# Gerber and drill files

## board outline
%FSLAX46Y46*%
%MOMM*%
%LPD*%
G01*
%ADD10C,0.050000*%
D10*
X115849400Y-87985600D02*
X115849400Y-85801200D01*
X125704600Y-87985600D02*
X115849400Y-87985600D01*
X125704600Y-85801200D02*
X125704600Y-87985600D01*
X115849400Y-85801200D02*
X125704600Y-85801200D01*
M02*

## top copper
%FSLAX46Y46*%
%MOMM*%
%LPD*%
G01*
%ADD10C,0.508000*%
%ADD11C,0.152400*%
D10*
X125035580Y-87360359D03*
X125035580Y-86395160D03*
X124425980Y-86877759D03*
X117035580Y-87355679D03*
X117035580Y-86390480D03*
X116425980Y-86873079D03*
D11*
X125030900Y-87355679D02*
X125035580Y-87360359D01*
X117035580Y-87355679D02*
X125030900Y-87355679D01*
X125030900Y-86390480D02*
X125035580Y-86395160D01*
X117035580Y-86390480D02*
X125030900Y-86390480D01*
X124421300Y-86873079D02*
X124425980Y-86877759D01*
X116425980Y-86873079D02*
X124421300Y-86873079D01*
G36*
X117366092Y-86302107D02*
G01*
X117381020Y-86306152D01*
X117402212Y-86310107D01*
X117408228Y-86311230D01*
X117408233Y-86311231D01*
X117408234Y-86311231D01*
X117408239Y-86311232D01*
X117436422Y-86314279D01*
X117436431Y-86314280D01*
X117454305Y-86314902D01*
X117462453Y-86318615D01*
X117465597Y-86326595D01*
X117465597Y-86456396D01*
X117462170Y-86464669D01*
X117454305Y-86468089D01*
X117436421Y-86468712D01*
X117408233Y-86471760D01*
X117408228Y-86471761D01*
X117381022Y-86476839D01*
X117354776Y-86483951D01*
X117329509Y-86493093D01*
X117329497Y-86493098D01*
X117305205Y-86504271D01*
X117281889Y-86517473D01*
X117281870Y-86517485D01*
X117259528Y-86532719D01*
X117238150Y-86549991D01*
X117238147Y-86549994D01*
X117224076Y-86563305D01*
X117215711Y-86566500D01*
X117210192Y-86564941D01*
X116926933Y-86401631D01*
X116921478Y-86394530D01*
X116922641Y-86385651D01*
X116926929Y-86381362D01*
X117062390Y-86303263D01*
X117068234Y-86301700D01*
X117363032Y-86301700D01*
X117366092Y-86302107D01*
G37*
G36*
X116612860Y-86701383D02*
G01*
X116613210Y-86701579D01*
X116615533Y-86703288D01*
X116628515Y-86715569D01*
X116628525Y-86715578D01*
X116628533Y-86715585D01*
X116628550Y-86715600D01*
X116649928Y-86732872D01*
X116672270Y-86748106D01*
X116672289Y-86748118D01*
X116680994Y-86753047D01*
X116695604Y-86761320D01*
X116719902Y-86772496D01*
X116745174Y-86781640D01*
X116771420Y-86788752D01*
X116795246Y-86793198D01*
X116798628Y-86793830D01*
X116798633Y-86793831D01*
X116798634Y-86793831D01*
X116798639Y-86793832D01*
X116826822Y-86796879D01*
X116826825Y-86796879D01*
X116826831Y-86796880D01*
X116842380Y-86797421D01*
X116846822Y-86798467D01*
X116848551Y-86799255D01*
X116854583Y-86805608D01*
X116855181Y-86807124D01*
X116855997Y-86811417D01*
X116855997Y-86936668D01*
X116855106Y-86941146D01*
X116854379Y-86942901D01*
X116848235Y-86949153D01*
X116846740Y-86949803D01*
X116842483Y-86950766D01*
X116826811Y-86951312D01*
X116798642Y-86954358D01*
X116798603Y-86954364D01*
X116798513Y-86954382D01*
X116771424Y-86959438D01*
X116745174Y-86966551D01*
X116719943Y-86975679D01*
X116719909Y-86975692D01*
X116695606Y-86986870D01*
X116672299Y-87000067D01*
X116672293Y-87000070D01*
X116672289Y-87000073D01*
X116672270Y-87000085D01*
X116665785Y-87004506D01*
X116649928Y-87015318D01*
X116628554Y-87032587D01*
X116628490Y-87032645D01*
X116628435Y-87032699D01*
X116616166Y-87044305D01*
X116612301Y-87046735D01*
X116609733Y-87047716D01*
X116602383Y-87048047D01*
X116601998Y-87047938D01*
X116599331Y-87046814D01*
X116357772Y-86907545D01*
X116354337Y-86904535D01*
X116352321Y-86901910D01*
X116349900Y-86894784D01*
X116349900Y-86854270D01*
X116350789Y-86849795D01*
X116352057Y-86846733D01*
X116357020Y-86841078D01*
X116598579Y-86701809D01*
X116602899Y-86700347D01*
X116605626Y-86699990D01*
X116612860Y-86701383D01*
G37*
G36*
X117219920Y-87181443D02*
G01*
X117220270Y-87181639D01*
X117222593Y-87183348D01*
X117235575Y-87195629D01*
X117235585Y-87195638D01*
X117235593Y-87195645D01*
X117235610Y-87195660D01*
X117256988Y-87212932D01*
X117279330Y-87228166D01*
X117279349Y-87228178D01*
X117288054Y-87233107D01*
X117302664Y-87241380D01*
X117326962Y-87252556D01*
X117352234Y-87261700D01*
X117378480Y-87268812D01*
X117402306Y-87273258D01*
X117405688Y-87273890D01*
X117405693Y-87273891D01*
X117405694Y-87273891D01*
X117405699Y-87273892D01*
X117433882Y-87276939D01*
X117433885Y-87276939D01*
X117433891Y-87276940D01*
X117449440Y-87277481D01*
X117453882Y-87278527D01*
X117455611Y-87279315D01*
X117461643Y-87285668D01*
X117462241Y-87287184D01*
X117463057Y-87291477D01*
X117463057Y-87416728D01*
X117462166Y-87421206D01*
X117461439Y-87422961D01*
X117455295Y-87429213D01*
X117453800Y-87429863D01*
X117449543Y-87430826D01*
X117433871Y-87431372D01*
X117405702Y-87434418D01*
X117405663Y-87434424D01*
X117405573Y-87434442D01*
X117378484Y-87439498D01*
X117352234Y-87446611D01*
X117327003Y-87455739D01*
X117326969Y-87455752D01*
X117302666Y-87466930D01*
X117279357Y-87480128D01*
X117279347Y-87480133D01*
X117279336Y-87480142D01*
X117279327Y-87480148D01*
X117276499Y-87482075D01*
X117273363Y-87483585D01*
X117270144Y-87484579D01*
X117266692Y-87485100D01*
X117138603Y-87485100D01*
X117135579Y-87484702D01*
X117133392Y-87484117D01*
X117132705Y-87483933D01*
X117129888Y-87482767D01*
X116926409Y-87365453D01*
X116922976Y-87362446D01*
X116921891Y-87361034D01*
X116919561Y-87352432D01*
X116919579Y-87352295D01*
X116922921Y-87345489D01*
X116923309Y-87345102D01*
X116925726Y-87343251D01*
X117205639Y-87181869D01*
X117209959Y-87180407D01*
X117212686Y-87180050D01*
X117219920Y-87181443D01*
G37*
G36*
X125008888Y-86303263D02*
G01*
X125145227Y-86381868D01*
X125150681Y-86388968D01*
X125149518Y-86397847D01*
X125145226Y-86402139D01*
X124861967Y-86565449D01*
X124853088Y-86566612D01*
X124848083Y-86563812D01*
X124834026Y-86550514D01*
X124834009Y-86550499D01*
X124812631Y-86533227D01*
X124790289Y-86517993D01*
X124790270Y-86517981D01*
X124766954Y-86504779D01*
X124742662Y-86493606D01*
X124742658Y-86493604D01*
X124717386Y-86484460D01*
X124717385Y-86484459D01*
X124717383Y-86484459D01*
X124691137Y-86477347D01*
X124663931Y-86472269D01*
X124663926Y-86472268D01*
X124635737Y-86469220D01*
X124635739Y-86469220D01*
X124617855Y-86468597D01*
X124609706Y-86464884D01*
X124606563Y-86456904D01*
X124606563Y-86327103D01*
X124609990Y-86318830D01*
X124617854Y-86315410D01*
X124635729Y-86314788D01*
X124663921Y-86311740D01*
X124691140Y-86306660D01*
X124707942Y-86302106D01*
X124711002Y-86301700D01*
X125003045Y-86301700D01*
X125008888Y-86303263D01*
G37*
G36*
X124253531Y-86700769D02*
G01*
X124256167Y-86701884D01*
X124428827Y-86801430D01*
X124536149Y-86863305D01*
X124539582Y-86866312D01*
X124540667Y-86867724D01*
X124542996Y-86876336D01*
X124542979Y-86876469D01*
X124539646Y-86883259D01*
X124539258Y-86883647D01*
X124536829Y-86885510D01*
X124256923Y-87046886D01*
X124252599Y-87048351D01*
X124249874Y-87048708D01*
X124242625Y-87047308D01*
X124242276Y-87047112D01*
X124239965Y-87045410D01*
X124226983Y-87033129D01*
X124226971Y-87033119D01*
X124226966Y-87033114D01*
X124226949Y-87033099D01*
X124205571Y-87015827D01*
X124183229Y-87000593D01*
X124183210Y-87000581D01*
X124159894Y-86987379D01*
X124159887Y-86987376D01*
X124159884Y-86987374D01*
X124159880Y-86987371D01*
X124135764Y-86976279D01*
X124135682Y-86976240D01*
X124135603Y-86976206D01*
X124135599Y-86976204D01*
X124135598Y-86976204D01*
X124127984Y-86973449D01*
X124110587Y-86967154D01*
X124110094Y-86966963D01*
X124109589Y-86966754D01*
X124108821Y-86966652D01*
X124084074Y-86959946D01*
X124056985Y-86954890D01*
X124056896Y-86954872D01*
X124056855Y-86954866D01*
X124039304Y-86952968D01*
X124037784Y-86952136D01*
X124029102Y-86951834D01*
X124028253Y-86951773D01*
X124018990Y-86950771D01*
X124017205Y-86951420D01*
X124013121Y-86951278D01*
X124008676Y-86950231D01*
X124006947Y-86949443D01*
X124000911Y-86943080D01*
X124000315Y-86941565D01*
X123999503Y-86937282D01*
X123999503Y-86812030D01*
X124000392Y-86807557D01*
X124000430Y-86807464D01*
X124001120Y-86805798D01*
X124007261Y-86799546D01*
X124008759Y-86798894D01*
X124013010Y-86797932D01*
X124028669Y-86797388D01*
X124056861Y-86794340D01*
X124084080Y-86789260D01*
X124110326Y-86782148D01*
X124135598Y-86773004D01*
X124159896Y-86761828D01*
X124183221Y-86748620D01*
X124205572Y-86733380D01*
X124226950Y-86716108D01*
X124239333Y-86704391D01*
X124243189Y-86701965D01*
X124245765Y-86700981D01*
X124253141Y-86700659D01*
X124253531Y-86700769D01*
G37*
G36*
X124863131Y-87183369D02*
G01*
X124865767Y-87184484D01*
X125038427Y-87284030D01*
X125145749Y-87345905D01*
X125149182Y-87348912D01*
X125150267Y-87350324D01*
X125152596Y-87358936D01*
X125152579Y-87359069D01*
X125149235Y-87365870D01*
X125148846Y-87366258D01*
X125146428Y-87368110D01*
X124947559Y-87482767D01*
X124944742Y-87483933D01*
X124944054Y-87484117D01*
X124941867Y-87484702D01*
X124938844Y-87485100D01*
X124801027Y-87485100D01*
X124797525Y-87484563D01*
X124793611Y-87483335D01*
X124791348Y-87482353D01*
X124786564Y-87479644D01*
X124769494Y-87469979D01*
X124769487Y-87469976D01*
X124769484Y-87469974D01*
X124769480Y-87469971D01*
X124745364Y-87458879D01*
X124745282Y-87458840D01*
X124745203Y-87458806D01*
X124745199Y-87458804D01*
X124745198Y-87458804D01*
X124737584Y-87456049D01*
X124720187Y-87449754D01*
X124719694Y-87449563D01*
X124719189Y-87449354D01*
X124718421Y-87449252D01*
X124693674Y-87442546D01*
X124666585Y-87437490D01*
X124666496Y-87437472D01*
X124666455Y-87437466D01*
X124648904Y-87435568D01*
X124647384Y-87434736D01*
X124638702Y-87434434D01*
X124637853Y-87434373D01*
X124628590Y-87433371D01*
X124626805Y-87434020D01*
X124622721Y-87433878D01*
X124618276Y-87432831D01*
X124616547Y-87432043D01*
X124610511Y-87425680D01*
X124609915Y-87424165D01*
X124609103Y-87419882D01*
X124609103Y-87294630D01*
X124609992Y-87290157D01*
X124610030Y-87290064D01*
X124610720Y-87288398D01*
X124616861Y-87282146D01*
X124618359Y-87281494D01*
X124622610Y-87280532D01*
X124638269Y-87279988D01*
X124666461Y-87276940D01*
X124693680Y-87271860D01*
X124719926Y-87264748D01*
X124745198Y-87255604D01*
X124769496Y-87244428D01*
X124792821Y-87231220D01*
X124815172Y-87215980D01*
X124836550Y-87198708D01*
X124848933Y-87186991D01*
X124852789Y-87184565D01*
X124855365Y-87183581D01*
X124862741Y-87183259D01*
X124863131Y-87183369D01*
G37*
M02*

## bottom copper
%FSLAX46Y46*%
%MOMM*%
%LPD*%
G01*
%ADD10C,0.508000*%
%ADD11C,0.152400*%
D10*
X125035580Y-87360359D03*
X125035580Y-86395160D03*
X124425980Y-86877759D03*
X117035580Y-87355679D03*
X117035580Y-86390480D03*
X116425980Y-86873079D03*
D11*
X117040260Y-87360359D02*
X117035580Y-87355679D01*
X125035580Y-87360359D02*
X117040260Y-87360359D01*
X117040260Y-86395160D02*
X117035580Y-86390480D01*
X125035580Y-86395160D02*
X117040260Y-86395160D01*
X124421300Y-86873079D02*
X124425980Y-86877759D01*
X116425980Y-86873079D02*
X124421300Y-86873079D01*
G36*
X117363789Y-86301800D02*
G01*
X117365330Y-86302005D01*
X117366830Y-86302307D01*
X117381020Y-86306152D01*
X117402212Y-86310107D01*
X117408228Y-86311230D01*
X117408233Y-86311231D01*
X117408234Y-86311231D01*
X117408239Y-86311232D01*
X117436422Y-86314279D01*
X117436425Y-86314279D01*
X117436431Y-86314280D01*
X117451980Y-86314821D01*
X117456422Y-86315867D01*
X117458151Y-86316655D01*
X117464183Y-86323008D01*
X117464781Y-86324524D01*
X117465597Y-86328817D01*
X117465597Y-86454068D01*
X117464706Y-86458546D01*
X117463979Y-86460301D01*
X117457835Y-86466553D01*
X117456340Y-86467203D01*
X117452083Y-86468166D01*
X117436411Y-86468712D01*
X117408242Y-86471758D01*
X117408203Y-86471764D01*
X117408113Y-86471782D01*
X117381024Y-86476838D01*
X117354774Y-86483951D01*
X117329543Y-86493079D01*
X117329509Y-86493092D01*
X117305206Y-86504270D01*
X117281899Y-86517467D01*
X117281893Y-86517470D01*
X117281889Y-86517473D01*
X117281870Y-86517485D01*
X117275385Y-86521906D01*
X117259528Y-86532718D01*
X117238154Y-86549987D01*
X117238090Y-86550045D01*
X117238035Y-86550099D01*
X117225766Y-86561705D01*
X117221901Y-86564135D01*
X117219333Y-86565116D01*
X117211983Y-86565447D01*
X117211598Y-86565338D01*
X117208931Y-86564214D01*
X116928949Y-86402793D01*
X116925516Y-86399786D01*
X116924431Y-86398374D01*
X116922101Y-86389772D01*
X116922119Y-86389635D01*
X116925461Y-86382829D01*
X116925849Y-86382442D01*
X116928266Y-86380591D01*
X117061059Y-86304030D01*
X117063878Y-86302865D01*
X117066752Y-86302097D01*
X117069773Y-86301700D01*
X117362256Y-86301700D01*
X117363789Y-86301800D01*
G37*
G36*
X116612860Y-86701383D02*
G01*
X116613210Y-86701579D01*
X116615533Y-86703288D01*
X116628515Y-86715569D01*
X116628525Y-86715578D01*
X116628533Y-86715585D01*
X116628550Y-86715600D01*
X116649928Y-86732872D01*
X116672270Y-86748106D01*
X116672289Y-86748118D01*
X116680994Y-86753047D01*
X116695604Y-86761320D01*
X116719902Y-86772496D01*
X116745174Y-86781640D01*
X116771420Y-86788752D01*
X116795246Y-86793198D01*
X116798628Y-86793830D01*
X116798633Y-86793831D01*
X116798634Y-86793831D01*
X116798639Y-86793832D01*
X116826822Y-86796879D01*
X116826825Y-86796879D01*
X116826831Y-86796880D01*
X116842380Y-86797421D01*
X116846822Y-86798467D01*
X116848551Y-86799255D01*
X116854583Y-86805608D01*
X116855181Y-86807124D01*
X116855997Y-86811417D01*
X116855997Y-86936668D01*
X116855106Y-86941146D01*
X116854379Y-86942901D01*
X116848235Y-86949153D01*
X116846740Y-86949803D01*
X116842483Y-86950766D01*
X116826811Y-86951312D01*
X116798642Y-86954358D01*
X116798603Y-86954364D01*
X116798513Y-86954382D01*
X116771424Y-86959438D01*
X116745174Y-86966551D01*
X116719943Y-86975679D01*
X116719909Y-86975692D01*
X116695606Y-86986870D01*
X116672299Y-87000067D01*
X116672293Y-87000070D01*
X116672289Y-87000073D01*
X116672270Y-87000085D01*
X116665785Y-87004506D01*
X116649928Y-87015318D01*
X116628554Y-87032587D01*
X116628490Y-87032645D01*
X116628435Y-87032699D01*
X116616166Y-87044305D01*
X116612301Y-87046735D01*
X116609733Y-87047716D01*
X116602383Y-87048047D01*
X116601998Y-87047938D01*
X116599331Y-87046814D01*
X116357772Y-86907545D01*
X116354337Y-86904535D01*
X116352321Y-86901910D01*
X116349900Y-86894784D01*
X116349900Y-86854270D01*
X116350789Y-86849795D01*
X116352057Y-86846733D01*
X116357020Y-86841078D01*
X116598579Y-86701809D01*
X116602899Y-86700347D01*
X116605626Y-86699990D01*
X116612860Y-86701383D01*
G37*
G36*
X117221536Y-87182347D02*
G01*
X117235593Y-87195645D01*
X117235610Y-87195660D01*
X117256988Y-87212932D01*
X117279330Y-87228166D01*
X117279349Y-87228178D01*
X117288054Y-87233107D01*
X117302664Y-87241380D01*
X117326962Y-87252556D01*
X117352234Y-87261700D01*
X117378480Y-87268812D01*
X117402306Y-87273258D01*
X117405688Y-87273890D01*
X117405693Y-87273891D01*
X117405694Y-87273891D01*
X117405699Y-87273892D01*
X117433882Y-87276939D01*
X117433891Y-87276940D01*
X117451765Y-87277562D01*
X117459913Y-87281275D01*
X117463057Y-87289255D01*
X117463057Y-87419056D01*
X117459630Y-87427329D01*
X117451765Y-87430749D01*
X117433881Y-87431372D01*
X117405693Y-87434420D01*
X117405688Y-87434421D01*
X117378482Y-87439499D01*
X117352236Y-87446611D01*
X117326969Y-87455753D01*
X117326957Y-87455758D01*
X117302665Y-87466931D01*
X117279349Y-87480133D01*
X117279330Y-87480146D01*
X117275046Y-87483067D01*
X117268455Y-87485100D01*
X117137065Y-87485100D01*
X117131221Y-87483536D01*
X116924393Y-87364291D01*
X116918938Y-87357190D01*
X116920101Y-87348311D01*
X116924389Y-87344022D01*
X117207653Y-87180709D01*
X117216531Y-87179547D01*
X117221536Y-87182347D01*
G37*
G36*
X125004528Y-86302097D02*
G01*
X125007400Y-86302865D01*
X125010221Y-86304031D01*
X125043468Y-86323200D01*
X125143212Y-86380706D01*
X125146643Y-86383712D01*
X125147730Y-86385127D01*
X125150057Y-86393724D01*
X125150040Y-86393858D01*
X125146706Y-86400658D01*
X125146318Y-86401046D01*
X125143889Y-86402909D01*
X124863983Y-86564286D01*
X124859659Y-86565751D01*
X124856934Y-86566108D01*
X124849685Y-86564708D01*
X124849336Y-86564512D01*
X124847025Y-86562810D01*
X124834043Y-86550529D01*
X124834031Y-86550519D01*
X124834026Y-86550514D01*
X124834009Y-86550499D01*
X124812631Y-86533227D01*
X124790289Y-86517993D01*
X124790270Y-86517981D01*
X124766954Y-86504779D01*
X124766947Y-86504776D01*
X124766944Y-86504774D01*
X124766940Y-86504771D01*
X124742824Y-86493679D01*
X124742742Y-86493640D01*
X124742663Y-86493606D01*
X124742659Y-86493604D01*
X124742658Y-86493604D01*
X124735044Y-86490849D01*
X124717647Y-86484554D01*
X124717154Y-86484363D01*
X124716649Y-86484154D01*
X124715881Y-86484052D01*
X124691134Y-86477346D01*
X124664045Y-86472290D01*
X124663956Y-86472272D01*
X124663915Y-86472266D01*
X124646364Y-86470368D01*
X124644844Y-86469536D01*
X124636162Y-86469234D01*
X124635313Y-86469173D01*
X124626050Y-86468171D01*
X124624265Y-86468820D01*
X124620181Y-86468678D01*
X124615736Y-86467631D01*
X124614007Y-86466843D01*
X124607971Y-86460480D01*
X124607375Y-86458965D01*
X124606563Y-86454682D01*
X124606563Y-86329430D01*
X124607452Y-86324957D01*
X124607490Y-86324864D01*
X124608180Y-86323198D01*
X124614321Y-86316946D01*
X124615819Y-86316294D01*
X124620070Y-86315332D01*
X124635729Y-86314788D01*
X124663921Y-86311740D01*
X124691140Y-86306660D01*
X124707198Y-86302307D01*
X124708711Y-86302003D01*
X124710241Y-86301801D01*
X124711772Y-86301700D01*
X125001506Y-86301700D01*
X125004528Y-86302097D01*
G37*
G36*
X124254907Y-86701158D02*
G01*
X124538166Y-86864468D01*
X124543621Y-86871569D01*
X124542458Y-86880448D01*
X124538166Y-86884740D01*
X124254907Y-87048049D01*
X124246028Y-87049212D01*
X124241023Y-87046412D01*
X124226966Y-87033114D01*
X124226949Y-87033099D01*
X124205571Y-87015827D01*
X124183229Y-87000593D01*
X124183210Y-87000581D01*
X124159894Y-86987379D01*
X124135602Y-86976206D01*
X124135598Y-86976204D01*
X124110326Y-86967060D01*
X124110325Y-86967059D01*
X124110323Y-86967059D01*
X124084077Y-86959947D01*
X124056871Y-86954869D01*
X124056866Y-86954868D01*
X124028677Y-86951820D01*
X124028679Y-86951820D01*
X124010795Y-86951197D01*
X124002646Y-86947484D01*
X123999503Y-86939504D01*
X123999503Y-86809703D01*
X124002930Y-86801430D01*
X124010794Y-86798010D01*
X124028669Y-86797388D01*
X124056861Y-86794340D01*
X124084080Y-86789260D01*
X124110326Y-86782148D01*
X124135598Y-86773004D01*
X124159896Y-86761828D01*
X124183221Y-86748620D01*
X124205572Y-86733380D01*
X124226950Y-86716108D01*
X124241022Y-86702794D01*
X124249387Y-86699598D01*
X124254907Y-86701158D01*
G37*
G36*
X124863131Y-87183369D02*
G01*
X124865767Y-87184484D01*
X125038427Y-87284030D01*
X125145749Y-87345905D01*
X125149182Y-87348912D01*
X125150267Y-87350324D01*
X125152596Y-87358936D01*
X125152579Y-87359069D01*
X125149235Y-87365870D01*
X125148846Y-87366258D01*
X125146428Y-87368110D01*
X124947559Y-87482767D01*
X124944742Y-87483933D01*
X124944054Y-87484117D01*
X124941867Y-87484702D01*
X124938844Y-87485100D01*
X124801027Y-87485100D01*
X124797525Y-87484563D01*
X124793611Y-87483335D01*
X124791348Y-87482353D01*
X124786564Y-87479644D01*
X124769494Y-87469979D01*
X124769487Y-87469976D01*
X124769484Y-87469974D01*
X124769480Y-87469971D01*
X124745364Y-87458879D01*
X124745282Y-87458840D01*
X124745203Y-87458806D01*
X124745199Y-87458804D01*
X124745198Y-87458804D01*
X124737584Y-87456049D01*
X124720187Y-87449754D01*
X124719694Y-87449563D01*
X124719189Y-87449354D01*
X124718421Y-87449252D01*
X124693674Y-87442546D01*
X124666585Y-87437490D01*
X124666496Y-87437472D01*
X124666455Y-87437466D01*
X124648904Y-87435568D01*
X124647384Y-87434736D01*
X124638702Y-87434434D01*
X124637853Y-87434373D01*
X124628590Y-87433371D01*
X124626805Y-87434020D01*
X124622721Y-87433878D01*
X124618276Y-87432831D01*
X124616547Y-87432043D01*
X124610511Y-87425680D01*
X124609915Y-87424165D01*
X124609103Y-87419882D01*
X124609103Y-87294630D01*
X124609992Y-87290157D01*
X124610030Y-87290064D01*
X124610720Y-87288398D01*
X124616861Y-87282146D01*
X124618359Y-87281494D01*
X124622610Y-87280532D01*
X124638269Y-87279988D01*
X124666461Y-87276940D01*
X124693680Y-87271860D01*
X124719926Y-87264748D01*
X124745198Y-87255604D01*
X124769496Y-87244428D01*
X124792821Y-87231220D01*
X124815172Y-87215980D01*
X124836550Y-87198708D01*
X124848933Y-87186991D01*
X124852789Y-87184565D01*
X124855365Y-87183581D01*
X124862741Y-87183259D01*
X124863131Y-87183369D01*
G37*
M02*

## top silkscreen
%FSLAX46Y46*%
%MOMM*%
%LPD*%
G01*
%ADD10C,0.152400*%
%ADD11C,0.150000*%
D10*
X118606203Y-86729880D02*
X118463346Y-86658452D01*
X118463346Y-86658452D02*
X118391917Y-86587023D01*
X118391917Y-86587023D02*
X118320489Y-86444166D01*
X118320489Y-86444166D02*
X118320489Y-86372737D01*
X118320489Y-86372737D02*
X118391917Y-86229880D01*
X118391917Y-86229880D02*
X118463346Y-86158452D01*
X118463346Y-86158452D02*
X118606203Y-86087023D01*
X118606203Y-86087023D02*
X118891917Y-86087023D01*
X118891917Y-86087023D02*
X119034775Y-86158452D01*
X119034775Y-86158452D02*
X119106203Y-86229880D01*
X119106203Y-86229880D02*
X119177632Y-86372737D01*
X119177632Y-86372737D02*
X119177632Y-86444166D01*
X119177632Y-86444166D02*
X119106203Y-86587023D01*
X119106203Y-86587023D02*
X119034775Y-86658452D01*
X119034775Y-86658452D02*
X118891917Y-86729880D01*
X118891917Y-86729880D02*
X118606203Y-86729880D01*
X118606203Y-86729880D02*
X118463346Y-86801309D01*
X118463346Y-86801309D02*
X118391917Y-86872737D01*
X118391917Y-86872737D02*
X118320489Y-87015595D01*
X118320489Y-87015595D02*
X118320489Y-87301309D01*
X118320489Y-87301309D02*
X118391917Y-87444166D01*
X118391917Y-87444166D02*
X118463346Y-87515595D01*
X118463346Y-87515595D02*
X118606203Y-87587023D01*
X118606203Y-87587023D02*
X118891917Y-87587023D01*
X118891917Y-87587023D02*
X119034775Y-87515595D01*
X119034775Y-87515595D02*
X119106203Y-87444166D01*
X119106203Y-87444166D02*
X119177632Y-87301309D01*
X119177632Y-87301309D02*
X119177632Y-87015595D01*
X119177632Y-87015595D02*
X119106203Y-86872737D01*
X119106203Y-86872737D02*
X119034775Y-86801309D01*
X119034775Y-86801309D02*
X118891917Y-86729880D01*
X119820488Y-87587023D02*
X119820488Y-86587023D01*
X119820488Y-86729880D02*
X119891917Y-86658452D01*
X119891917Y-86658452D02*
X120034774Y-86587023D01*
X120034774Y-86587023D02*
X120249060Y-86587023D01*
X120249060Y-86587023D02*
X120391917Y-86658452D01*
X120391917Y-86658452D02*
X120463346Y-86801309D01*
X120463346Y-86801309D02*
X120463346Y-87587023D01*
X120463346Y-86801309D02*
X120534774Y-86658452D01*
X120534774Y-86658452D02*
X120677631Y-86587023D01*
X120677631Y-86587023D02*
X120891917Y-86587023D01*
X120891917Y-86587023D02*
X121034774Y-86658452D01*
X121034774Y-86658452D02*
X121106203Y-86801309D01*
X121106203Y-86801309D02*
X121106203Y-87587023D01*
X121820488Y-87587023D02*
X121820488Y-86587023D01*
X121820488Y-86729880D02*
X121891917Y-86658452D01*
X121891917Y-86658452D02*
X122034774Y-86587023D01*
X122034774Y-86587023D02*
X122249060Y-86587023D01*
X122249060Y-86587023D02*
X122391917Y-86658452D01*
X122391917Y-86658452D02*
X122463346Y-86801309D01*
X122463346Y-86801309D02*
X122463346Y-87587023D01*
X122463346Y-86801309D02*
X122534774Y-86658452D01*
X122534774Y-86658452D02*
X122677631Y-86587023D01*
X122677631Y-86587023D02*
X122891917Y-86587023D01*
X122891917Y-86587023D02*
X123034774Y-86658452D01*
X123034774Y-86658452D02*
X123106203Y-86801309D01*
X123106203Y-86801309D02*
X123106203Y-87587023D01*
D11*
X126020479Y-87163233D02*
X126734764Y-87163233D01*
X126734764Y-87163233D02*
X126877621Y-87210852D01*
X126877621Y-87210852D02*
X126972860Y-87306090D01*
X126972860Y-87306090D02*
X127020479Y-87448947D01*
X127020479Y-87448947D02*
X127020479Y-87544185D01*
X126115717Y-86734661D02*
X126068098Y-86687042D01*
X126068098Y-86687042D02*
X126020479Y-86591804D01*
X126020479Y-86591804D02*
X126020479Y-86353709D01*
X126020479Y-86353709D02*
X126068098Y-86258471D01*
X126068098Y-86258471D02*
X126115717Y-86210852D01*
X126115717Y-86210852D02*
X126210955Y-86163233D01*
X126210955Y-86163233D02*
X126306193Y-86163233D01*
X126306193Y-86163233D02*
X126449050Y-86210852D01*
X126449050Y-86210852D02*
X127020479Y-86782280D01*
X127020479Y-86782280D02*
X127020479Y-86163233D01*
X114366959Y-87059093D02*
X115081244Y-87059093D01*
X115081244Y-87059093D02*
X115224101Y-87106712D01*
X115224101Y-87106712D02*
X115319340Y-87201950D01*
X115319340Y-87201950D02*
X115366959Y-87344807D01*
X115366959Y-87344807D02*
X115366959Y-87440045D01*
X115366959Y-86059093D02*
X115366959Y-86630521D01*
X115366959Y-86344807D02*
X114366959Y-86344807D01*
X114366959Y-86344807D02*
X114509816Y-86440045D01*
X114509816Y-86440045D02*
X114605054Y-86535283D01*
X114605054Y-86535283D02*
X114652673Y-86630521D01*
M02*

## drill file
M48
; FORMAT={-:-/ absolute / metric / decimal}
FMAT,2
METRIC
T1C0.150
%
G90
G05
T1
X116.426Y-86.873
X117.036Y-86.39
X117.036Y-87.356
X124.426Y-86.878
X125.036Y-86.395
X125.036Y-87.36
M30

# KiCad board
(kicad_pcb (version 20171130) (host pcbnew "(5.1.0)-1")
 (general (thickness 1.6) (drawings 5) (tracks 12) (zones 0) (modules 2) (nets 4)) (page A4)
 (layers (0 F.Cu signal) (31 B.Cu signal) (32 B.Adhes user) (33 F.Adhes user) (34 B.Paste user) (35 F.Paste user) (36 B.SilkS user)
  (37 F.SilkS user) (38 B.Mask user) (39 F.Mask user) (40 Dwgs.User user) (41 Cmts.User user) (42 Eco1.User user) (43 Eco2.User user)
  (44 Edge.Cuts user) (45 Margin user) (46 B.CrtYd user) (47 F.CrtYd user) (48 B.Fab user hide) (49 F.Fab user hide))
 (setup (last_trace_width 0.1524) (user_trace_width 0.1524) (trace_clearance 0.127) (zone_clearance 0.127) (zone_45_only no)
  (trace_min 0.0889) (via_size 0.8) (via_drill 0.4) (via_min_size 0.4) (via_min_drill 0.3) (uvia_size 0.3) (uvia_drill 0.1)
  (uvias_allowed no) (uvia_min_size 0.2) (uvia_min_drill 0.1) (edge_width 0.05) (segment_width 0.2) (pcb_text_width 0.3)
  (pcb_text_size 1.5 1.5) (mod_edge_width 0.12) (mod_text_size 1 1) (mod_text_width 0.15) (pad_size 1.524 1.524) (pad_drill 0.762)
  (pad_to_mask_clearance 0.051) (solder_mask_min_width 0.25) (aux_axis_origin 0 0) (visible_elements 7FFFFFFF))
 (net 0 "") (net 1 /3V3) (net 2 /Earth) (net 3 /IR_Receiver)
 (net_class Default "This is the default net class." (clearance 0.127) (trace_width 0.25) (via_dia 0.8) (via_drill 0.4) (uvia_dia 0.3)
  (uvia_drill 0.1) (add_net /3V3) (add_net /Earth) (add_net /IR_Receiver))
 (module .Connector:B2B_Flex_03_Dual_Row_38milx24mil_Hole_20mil (layer F.Cu) (at 125.01058 86.37016 270)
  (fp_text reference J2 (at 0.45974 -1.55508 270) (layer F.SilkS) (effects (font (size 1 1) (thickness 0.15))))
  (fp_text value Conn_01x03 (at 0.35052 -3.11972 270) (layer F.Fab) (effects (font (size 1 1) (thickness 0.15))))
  (pad 3 thru_hole circle (at 0.990199 -0.025 270) (size 0.508 0.508) (drill 0.15) (layers *.Cu *.Mask) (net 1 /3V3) (zone_connect 2))
  (pad 1 thru_hole circle (at 0.025 -0.025 270) (size 0.508 0.508) (drill 0.15) (layers *.Cu *.Mask) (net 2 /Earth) (zone_connect 2))
  (pad 2 thru_hole circle (at 0.507599 0.5846 270) (size 0.508 0.508) (drill 0.15) (layers *.Cu *.Mask) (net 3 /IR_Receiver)
   (zone_connect 2)))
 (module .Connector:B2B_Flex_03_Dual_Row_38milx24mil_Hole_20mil (layer F.Cu) (at 117.01058 86.36548 270)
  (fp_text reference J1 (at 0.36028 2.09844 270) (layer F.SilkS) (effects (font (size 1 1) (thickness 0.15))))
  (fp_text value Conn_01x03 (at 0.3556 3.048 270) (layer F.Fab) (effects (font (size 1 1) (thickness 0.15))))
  (pad 3 thru_hole circle (at 0.990199 -0.025 270) (size 0.508 0.508) (drill 0.15) (layers *.Cu *.Mask) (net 1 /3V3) (zone_connect 2))
  (pad 1 thru_hole circle (at 0.025 -0.025 270) (size 0.508 0.508) (drill 0.15) (layers *.Cu *.Mask) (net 2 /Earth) (zone_connect 2))
  (pad 2 thru_hole circle (at 0.507599 0.5846 270) (size 0.508 0.508) (drill 0.15) (layers *.Cu *.Mask) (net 3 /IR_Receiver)
   (zone_connect 2)))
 (gr_line (start 115.8494 87.9856) (end 115.8494 85.8012) (layer Edge.Cuts) (width 0.05))
 (gr_line (start 125.7046 87.9856) (end 115.8494 87.9856) (layer Edge.Cuts) (width 0.05))
 (gr_line (start 125.7046 85.8012) (end 125.7046 87.9856) (layer Edge.Cuts) (width 0.05))
 (gr_line (start 115.8494 85.8012) (end 125.7046 85.8012) (layer Edge.Cuts) (width 0.05))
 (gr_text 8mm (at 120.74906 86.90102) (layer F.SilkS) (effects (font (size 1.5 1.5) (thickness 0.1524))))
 (segment (start 125.0309 87.355679) (end 125.03558 87.360359) (width 0.1524) (layer F.Cu) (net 1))
 (segment (start 117.03558 87.355679) (end 125.0309 87.355679) (width 0.1524) (layer F.Cu) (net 1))
 (segment (start 117.04026 87.360359) (end 117.03558 87.355679) (width 0.1524) (layer B.Cu) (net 1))
 (segment (start 125.03558 87.360359) (end 117.04026 87.360359) (width 0.1524) (layer B.Cu) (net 1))
 (segment (start 125.0309 86.39048) (end 125.03558 86.39516) (width 0.1524) (layer F.Cu) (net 2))
 (segment (start 117.03558 86.39048) (end 125.0309 86.39048) (width 0.1524) (layer F.Cu) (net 2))
 (segment (start 117.04026 86.39516) (end 117.03558 86.39048) (width 0.1524) (layer B.Cu) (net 2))
 (segment (start 125.03558 86.39516) (end 117.04026 86.39516) (width 0.1524) (layer B.Cu) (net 2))
 (segment (start 124.4213 86.873079) (end 124.42598 86.877759) (width 0.1524) (layer F.Cu) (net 3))
 (segment (start 116.42598 86.873079) (end 124.4213 86.873079) (width 0.1524) (layer F.Cu) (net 3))
 (segment (start 124.4213 86.873079) (end 124.42598 86.877759) (width 0.1524) (layer B.Cu) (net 3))
 (segment (start 116.42598 86.873079) (end 124.4213 86.873079) (width 0.1524) (layer B.Cu) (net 3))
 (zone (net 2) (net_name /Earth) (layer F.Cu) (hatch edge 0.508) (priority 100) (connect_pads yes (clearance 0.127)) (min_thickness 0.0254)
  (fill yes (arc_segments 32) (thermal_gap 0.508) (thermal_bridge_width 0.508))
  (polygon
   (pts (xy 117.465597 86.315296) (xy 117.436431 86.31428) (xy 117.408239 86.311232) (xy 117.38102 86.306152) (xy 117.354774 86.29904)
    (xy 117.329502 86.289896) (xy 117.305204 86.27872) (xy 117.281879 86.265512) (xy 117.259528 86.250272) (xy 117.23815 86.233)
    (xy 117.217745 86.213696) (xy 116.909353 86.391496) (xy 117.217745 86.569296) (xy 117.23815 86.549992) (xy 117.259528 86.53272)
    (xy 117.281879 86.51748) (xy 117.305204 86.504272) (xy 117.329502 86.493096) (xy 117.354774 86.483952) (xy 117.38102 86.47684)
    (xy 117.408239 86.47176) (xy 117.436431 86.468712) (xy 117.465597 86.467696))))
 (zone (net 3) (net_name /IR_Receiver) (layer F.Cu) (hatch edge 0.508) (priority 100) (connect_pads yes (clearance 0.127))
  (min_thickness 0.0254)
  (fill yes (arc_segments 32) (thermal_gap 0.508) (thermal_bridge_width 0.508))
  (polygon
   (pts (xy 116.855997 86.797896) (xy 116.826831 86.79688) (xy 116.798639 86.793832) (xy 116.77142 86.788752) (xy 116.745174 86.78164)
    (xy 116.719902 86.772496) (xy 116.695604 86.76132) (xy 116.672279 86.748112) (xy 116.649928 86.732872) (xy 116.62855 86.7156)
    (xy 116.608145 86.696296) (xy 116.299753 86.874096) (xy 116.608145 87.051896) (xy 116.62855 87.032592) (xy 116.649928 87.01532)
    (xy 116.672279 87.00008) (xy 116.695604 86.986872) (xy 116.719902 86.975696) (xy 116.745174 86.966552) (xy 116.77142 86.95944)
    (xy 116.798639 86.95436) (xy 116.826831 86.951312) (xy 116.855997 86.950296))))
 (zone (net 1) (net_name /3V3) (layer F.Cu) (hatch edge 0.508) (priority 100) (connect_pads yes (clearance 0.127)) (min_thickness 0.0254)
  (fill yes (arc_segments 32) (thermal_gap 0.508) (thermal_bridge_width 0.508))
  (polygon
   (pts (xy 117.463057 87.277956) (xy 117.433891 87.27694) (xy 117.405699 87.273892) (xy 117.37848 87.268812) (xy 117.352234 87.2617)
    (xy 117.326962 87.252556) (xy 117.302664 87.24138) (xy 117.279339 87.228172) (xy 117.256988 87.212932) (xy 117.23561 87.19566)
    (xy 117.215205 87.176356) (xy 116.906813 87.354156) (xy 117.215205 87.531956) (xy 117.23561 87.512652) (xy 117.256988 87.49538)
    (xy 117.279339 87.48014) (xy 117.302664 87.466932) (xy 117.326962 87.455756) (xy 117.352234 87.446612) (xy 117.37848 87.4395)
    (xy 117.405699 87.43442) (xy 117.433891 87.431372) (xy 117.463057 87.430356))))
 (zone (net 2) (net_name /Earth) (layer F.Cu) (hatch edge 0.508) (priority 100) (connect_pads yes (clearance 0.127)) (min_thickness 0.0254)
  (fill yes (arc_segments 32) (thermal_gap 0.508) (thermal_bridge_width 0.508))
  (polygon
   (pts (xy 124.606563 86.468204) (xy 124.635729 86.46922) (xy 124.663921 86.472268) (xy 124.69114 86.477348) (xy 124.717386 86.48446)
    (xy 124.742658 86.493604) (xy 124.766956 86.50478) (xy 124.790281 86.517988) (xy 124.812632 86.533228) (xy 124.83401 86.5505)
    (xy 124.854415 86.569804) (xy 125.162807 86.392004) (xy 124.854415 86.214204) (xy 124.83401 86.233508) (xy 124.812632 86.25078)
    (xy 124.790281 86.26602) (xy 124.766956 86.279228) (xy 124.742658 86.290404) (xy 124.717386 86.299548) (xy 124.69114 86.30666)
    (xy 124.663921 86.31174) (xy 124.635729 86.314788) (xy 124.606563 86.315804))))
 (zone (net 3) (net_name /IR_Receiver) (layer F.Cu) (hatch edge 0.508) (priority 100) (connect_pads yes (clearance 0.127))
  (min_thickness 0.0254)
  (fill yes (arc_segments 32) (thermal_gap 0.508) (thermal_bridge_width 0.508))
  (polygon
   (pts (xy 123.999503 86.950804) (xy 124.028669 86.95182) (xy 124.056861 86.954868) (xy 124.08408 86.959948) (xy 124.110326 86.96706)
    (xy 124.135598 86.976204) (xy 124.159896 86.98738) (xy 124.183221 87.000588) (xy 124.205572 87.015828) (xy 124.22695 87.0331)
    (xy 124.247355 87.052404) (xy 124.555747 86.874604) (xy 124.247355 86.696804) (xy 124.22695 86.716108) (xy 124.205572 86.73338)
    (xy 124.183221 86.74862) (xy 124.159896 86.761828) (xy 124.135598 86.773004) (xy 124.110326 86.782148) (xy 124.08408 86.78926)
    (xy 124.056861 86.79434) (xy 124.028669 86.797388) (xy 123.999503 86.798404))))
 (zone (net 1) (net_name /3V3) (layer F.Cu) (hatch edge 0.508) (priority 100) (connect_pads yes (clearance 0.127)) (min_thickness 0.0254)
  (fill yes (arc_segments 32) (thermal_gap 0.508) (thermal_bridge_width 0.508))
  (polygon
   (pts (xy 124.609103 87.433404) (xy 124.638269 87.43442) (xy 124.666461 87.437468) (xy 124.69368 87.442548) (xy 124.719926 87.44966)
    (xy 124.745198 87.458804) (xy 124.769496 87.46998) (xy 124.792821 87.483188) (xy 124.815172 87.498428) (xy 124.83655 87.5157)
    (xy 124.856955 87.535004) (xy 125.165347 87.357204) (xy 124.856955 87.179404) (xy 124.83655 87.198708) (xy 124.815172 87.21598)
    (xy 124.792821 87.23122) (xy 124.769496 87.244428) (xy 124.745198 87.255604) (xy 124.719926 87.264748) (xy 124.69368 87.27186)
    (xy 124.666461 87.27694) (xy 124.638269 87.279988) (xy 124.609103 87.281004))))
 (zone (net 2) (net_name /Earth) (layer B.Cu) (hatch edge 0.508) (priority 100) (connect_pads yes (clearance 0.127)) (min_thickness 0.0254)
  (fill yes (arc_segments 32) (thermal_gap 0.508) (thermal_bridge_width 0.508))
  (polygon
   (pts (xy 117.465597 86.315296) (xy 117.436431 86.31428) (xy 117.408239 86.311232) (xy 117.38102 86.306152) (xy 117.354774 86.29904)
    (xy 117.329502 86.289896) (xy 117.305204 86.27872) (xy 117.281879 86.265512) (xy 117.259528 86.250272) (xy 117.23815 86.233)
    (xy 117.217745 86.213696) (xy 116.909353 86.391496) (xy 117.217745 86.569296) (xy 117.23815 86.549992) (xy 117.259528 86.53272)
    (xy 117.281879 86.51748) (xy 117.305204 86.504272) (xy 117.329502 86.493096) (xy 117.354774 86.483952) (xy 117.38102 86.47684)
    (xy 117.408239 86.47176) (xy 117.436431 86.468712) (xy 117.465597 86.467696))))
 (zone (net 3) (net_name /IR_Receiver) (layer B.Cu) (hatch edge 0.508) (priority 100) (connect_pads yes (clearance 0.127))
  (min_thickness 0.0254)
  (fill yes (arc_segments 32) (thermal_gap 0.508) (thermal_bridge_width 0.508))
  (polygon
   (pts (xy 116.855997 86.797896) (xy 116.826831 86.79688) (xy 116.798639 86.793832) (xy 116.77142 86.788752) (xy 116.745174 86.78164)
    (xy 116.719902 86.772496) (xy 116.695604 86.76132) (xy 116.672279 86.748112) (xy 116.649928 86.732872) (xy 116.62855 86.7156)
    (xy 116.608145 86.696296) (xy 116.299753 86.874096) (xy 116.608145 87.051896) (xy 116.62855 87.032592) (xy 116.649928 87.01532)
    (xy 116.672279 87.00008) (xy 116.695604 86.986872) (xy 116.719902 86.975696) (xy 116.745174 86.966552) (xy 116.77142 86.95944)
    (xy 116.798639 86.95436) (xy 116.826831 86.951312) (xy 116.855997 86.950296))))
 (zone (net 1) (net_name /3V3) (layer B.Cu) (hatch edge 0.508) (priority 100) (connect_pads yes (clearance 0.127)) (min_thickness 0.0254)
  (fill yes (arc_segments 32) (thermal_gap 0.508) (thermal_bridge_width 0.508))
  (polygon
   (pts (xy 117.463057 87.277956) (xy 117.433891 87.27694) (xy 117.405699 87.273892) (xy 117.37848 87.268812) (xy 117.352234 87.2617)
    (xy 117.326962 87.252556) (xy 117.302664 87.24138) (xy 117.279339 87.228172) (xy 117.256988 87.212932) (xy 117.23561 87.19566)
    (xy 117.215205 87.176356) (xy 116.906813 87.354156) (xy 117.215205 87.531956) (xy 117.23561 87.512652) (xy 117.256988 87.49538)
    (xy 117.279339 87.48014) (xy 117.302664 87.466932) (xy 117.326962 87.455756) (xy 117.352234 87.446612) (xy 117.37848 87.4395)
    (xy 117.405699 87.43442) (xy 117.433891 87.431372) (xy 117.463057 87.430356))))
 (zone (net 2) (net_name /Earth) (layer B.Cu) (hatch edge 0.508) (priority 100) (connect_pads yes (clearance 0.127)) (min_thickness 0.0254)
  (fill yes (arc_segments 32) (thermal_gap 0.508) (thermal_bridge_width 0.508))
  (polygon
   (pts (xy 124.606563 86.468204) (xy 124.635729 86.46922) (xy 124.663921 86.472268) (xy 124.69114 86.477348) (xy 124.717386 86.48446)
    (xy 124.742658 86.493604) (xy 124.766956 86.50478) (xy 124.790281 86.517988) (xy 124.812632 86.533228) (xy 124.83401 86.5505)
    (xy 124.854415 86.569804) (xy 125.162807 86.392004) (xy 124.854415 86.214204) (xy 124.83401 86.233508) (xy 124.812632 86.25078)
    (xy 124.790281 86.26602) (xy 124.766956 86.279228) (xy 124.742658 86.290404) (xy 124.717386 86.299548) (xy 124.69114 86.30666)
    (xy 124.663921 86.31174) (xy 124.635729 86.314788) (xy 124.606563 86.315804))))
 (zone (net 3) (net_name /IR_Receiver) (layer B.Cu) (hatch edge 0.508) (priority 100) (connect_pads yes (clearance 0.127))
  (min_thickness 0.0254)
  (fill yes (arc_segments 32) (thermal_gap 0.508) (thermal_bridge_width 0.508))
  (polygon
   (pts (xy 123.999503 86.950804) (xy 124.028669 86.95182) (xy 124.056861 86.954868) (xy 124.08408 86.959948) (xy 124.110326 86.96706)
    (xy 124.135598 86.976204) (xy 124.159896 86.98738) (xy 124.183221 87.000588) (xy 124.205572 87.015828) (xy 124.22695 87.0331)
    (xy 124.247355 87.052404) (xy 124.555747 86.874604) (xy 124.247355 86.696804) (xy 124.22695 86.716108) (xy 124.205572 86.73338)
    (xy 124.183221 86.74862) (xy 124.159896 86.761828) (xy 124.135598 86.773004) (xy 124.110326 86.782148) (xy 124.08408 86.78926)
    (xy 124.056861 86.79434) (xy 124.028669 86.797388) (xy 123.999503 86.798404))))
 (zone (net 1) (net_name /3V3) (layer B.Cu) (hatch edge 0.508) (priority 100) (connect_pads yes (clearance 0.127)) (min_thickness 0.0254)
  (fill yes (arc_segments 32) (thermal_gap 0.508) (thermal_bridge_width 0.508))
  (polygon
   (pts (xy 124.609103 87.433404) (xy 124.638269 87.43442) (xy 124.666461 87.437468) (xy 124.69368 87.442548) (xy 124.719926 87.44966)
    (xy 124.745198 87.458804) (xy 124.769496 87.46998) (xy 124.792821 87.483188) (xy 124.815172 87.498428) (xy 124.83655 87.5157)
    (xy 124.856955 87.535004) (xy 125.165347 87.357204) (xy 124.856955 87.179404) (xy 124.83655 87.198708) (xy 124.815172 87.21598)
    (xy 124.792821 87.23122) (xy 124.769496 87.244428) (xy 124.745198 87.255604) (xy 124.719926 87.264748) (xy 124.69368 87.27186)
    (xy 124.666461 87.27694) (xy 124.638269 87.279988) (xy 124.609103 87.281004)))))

